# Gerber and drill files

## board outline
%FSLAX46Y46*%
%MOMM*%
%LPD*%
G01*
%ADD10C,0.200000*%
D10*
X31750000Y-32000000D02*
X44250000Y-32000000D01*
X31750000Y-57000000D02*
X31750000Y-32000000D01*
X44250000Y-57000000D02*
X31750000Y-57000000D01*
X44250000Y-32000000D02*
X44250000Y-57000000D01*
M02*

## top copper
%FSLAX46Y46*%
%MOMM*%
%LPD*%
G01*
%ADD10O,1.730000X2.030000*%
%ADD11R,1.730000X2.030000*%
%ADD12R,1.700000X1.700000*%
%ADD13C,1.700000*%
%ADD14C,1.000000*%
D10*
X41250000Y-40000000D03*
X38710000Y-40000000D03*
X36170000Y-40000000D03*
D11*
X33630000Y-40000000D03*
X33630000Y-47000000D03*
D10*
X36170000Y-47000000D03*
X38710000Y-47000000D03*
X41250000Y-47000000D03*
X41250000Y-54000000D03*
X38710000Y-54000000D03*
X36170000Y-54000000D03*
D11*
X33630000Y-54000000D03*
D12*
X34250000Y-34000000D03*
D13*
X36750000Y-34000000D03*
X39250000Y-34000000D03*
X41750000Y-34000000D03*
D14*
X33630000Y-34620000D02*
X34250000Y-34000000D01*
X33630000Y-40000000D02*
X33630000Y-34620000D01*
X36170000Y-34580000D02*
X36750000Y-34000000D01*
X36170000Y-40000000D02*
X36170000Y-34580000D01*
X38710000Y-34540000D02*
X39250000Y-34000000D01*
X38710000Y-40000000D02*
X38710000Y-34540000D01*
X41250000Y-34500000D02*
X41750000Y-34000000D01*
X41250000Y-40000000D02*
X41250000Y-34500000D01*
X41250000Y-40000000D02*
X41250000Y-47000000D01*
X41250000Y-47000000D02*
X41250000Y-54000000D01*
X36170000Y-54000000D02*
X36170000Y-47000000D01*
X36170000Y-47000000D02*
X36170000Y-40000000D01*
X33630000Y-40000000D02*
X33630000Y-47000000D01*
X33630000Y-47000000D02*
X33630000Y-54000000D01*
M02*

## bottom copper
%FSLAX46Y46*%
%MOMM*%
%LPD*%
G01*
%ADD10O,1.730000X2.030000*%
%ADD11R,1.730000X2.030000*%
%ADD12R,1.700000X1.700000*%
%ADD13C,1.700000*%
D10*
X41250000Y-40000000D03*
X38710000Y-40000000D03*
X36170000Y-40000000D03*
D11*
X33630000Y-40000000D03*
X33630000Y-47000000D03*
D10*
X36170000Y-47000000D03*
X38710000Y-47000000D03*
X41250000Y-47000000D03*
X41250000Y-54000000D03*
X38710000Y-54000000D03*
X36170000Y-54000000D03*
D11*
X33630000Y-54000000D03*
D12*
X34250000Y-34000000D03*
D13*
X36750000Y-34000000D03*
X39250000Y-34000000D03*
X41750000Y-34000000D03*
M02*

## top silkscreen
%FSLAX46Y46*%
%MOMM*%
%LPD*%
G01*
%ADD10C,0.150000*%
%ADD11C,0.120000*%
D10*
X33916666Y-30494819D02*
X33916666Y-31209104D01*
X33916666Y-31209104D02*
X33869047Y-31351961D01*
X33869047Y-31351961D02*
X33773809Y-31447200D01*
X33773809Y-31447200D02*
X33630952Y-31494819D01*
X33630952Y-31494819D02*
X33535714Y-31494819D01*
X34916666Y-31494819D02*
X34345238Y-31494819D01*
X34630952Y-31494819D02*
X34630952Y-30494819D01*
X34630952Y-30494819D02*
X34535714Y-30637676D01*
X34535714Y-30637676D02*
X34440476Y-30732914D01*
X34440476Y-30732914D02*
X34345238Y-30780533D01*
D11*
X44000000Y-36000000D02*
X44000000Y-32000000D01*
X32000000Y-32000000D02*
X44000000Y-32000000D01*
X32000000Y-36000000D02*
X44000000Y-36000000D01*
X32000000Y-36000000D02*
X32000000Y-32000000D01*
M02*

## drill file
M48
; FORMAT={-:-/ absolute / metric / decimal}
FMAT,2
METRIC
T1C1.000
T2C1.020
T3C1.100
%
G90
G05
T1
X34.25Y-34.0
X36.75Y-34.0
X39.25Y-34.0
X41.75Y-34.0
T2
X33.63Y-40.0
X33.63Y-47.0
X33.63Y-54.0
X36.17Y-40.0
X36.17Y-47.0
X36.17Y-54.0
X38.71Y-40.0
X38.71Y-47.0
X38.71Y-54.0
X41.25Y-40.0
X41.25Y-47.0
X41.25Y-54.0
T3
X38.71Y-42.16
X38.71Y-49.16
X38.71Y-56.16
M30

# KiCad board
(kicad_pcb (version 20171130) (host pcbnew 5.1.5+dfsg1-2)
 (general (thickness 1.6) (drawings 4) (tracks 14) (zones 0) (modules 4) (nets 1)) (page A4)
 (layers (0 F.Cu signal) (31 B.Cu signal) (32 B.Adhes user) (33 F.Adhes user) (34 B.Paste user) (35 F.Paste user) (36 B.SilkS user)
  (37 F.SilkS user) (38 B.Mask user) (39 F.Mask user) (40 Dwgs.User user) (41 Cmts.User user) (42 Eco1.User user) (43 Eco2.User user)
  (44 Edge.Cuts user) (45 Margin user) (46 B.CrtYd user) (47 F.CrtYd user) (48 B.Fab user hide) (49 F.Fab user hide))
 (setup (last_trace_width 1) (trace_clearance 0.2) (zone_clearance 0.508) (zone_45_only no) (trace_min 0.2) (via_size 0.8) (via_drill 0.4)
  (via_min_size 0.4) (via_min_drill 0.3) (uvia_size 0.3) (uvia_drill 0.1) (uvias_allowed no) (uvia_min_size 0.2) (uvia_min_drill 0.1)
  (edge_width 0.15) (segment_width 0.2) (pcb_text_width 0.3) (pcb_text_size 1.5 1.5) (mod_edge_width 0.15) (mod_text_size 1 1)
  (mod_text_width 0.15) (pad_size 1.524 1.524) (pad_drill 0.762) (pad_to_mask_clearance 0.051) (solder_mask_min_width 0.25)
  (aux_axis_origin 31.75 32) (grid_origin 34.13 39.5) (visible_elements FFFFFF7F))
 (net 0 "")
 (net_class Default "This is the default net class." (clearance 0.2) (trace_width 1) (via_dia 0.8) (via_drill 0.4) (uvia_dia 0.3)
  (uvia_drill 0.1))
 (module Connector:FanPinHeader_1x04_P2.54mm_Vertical (layer B.Cu) (at 33.63 40)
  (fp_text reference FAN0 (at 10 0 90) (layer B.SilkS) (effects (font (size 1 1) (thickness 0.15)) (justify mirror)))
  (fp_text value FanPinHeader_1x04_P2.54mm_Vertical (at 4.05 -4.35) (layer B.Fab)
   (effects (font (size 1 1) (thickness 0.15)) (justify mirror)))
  (pad "" np_thru_hole circle (at 5.08 2.16 270) (size 1.1 1.1) (drill 1.1) (layers *.Cu *.Mask))
  (pad 4 thru_hole oval (at 7.62 0 270) (size 2.03 1.73) (drill 1.02) (layers *.Cu *.Mask))
  (pad 3 thru_hole oval (at 5.08 0 270) (size 2.03 1.73) (drill 1.02) (layers *.Cu *.Mask))
  (pad 2 thru_hole oval (at 2.54 0 270) (size 2.03 1.73) (drill 1.02) (layers *.Cu *.Mask))
  (pad 1 thru_hole rect (at 0 0 270) (size 2.03 1.73) (drill 1.02) (layers *.Cu *.Mask)))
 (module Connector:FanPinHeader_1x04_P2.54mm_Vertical (layer B.Cu) (at 33.63 47)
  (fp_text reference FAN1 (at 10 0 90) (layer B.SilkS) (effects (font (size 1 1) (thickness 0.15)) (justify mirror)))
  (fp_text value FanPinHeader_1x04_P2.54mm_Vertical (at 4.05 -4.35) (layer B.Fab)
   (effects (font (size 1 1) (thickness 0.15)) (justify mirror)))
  (pad 1 thru_hole rect (at 0 0 270) (size 2.03 1.73) (drill 1.02) (layers *.Cu *.Mask))
  (pad 2 thru_hole oval (at 2.54 0 270) (size 2.03 1.73) (drill 1.02) (layers *.Cu *.Mask))
  (pad 3 thru_hole oval (at 5.08 0 270) (size 2.03 1.73) (drill 1.02) (layers *.Cu *.Mask))
  (pad 4 thru_hole oval (at 7.62 0 270) (size 2.03 1.73) (drill 1.02) (layers *.Cu *.Mask))
  (pad "" np_thru_hole circle (at 5.08 2.16 270) (size 1.1 1.1) (drill 1.1) (layers *.Cu *.Mask)))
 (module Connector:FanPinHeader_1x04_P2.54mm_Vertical (layer B.Cu) (at 33.63 54)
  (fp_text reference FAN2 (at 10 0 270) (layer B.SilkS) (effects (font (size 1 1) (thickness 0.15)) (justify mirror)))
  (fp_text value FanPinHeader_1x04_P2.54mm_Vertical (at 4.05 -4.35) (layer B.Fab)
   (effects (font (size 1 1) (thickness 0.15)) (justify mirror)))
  (pad "" np_thru_hole circle (at 5.08 2.16 270) (size 1.1 1.1) (drill 1.1) (layers *.Cu *.Mask))
  (pad 4 thru_hole oval (at 7.62 0 270) (size 2.03 1.73) (drill 1.02) (layers *.Cu *.Mask))
  (pad 3 thru_hole oval (at 5.08 0 270) (size 2.03 1.73) (drill 1.02) (layers *.Cu *.Mask))
  (pad 2 thru_hole oval (at 2.54 0 270) (size 2.03 1.73) (drill 1.02) (layers *.Cu *.Mask))
  (pad 1 thru_hole rect (at 0 0 270) (size 2.03 1.73) (drill 1.02) (layers *.Cu *.Mask)))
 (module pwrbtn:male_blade (layer F.Cu) (at 38 34)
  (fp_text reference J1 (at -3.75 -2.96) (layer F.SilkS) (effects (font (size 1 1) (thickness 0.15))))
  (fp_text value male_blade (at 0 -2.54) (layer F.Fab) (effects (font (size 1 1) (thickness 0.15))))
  (fp_line (start 6 2) (end 6 -2) (layer F.SilkS) (width 0.12))
  (fp_line (start -6 -2) (end 6 -2) (layer F.SilkS) (width 0.12))
  (fp_line (start -6 2) (end 6 2) (layer F.SilkS) (width 0.12))
  (fp_line (start -6 2) (end -6 -2) (layer F.SilkS) (width 0.12))
  (pad 1 thru_hole rect (at -3.75 0 90) (size 1.7 1.7) (drill 1) (layers *.Cu *.Mask))
  (pad 2 thru_hole circle (at -1.25 0 90) (size 1.7 1.7) (drill 1) (layers *.Cu *.Mask))
  (pad 3 thru_hole circle (at 1.25 0 90) (size 1.7 1.7) (drill 1) (layers *.Cu *.Mask))
  (pad 4 thru_hole circle (at 3.75 0 90) (size 1.7 1.7) (drill 1) (layers *.Cu *.Mask)))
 (gr_line (start 31.75 32) (end 44.25 32) (layer Edge.Cuts) (width 0.2))
 (gr_line (start 31.75 57) (end 31.75 32) (layer Edge.Cuts) (width 0.2))
 (gr_line (start 44.25 57) (end 31.75 57) (layer Edge.Cuts) (width 0.2))
 (gr_line (start 44.25 32) (end 44.25 57) (layer Edge.Cuts) (width 0.2))
 (segment (start 33.63 34.62) (end 34.25 34) (width 1) (layer F.Cu) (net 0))
 (segment (start 33.63 40) (end 33.63 34.62) (width 1) (layer F.Cu) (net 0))
 (segment (start 36.17 34.58) (end 36.75 34) (width 1) (layer F.Cu) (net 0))
 (segment (start 36.17 40) (end 36.17 34.58) (width 1) (layer F.Cu) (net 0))
 (segment (start 38.71 34.54) (end 39.25 34) (width 1) (layer F.Cu) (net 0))
 (segment (start 38.71 40) (end 38.71 34.54) (width 1) (layer F.Cu) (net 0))
 (segment (start 41.25 34.5) (end 41.75 34) (width 1) (layer F.Cu) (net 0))
 (segment (start 41.25 40) (end 41.25 34.5) (width 1) (layer F.Cu) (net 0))
 (segment (start 41.25 40) (end 41.25 47) (width 1) (layer F.Cu) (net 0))
 (segment (start 41.25 47) (end 41.25 54) (width 1) (layer F.Cu) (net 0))
 (segment (start 36.17 54) (end 36.17 47) (width 1) (layer F.Cu) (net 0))
 (segment (start 36.17 47) (end 36.17 40) (width 1) (layer F.Cu) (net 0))
 (segment (start 33.63 40) (end 33.63 47) (width 1) (layer F.Cu) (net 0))
 (segment (start 33.63 47) (end 33.63 54) (width 1) (layer F.Cu) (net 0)))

